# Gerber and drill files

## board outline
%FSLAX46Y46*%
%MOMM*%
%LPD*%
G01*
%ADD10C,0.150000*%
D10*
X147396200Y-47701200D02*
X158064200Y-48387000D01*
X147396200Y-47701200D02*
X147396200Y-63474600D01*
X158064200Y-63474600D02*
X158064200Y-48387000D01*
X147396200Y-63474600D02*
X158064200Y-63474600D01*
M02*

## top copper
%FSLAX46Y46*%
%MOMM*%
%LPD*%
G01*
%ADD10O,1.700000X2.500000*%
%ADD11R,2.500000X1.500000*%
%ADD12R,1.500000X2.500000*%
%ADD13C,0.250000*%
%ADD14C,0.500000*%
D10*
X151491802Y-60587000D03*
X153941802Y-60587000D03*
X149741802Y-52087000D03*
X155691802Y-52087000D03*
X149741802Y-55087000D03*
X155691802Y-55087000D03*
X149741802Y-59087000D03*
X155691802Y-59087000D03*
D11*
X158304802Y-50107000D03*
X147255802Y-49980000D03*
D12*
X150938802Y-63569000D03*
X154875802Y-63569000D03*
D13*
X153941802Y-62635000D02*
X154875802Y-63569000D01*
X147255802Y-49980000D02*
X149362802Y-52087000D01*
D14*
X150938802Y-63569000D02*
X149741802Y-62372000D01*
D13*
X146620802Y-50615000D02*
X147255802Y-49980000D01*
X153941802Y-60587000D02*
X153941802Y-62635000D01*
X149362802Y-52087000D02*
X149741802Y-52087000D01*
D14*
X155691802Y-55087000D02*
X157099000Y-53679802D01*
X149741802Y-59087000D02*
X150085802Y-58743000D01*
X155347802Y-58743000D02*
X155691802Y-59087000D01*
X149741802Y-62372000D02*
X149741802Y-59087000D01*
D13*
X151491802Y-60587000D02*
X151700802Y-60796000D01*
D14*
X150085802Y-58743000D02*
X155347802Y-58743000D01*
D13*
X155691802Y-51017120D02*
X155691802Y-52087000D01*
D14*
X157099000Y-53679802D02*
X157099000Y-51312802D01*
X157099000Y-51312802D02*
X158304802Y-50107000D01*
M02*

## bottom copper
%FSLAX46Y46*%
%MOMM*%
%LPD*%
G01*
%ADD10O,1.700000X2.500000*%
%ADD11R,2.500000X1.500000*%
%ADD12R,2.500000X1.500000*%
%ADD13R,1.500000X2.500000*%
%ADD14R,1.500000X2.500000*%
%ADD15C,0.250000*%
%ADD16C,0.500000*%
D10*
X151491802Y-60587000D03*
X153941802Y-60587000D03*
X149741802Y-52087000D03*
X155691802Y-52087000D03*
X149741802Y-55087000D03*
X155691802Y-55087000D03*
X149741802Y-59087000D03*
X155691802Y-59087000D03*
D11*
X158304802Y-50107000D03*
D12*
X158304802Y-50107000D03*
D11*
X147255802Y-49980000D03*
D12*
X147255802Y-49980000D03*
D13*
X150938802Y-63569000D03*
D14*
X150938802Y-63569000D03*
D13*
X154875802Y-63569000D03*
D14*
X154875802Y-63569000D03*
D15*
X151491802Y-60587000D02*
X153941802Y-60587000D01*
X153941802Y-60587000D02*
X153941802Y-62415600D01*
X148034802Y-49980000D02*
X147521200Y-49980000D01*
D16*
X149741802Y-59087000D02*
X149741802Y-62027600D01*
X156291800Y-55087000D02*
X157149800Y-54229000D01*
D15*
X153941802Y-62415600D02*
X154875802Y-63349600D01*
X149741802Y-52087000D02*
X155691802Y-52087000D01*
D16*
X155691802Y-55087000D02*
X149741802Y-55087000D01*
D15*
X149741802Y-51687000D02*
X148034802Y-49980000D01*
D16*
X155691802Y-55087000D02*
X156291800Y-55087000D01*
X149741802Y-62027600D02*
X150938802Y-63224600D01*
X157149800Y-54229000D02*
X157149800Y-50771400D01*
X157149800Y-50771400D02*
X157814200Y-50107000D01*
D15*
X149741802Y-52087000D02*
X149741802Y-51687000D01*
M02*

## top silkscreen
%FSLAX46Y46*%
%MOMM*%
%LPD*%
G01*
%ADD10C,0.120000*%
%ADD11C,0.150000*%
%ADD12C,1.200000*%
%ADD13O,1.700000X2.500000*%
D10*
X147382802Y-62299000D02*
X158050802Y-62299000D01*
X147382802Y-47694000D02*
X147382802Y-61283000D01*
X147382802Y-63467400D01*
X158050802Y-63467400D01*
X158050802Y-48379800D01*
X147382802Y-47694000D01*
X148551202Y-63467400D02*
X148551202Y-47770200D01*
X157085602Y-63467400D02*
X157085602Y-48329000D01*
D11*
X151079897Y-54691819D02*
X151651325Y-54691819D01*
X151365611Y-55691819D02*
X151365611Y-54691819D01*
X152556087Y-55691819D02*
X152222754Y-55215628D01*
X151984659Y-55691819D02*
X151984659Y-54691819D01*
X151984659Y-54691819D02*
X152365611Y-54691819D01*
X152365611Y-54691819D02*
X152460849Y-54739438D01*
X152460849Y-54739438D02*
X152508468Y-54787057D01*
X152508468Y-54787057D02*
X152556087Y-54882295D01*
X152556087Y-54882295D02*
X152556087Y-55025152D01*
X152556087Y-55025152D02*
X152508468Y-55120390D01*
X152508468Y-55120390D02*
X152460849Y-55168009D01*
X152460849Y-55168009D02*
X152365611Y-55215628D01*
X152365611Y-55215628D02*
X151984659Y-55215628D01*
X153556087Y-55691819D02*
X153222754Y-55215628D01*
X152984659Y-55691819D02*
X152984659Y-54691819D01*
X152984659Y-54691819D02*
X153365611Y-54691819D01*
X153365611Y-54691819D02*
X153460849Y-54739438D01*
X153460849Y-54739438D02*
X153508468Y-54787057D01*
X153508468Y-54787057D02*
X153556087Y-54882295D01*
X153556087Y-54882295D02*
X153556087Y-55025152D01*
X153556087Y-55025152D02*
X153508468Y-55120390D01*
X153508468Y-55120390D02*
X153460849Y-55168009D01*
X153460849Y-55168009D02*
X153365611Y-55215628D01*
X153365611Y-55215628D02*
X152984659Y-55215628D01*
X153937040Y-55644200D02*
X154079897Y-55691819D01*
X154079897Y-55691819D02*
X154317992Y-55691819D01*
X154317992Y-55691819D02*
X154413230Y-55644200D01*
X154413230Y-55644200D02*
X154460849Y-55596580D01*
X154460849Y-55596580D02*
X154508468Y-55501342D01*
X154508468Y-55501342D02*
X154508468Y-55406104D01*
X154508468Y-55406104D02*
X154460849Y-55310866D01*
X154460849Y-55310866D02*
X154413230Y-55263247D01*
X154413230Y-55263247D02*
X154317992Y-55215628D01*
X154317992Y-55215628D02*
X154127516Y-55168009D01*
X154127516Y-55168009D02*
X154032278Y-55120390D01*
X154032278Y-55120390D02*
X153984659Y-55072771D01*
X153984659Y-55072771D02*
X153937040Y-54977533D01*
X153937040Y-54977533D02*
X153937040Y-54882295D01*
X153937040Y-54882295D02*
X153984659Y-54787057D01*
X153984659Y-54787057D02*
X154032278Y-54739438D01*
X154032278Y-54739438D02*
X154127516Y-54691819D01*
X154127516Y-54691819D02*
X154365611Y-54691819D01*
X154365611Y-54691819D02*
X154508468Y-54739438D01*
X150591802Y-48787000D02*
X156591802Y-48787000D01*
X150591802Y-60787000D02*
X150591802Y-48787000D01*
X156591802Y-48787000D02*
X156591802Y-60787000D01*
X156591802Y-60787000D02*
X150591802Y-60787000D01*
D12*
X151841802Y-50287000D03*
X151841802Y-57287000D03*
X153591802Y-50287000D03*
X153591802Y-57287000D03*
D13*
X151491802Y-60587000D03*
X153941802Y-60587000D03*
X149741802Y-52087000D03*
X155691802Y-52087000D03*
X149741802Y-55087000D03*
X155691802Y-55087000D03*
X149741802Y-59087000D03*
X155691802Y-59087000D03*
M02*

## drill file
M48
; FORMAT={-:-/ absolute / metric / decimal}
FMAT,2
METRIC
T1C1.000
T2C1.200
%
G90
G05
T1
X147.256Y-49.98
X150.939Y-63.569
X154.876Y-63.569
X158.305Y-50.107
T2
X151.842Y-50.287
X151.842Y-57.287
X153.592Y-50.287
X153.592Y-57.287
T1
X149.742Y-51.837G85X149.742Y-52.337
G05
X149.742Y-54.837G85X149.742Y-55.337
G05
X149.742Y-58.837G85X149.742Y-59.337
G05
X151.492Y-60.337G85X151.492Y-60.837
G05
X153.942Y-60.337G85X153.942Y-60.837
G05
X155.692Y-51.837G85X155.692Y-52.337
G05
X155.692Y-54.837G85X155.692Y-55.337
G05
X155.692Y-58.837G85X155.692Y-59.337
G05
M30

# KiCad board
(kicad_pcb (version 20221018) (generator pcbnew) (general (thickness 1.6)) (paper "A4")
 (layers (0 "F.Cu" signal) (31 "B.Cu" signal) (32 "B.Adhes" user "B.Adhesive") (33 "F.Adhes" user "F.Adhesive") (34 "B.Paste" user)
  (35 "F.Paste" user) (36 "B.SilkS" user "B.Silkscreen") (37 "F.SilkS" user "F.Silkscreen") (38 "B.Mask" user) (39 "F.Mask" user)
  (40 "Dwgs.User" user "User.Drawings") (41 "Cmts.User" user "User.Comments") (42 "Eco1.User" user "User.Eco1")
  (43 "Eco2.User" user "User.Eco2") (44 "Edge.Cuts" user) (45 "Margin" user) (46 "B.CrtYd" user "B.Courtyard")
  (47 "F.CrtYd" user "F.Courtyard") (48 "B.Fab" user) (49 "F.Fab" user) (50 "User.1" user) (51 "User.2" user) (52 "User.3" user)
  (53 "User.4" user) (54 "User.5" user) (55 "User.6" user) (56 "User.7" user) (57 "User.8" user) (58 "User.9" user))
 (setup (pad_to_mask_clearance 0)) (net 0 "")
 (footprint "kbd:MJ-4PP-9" (layer "F.Cu") (at 153.591802 48.787)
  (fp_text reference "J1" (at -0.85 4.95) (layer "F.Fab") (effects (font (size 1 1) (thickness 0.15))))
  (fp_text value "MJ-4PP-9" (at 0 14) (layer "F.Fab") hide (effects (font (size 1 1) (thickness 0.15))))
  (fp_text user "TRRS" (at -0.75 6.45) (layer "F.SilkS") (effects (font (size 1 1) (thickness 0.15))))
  (fp_line (start -3 0) (end 3 0) (stroke (width 0.15) (type solid)) (layer "F.SilkS"))
  (fp_line (start -3 12) (end -3 0) (stroke (width 0.15) (type solid)) (layer "F.SilkS"))
  (fp_line (start 3 0) (end 3 12) (stroke (width 0.15) (type solid)) (layer "F.SilkS"))
  (fp_line (start 3 12) (end -3 12) (stroke (width 0.15) (type solid)) (layer "F.SilkS"))
  (pad "" np_thru_hole circle (at -1.75 1.5) (size 1.2 1.2) (drill 1.2) (layers "F&B.Cu" "*.Mask" "F.SilkS"))
  (pad "" np_thru_hole circle (at -1.75 8.5) (size 1.2 1.2) (drill 1.2) (layers "F&B.Cu" "*.Mask" "F.SilkS"))
  (pad "" np_thru_hole circle (at 0 1.5) (size 1.2 1.2) (drill 1.2) (layers "F&B.Cu" "*.Mask" "F.SilkS"))
  (pad "" np_thru_hole circle (at 0 8.5) (size 1.2 1.2) (drill 1.2) (layers "F&B.Cu" "*.Mask" "F.SilkS"))
  (pad "A" thru_hole oval (at -2.1 11.8) (size 1.7 2.5) (drill oval 1 1.5) (layers "*.Cu" "*.Mask" "F.SilkS") (clearance 0.15))
  (pad "A" thru_hole oval (at 0.35 11.8) (size 1.7 2.5) (drill oval 1 1.5) (layers "*.Cu" "*.Mask" "F.SilkS") (clearance 0.15))
  (pad "B" thru_hole oval (at -3.85 3.3) (size 1.7 2.5) (drill oval 1 1.5) (layers "*.Cu" "*.Mask" "F.SilkS"))
  (pad "B" thru_hole oval (at 2.1 3.3) (size 1.7 2.5) (drill oval 1 1.5) (layers "*.Cu" "*.Mask" "F.SilkS"))
  (pad "C" thru_hole oval (at -3.85 6.3) (size 1.7 2.5) (drill oval 1 1.5) (layers "*.Cu" "*.Mask" "F.SilkS"))
  (pad "C" thru_hole oval (at 2.1 6.3) (size 1.7 2.5) (drill oval 1 1.5) (layers "*.Cu" "*.Mask" "F.SilkS"))
  (pad "D" thru_hole oval (at -3.85 10.3) (size 1.7 2.5) (drill oval 1 1.5) (layers "*.Cu" "*.Mask" "F.SilkS") (clearance 0.15))
  (pad "D" thru_hole oval (at 2.1 10.3) (size 1.7 2.5) (drill oval 1 1.5) (layers "*.Cu" "*.Mask" "F.SilkS") (clearance 0.15)))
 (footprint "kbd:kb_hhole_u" (layer "F.Cu") (at 158.304802 50.107 -90)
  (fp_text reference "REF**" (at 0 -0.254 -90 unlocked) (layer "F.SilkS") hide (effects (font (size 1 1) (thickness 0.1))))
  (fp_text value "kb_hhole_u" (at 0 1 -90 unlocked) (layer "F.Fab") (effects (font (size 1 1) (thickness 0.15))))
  (pad "1" thru_hole rect (at 0 0 270) (size 1.5 2.5) (drill 1) (layers "*.Cu" "*.Adhes" "*.Mask"))
  (pad "1" smd rect (at 0 0 270) (size 1.5 2.5) (layers "*.Paste" "*.Mask" "B.Cu")))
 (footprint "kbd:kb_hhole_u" (layer "F.Cu") (at 147.255802 49.98 -90)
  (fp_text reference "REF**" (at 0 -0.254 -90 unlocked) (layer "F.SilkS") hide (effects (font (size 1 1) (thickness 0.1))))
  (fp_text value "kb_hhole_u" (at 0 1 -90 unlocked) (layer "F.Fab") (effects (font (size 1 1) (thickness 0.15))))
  (pad "1" thru_hole rect (at 0 0 270) (size 1.5 2.5) (drill 1) (layers "*.Cu" "*.Adhes" "*.Mask"))
  (pad "1" smd rect (at 0 0 270) (size 1.5 2.5) (layers "*.Paste" "*.Mask" "B.Cu")))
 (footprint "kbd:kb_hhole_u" (layer "F.Cu") (at 150.938802 63.569)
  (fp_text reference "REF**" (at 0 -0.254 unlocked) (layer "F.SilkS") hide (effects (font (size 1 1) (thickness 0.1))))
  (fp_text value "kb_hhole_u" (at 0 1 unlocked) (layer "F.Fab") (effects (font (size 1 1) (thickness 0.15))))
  (pad "1" thru_hole rect (at 0 0) (size 1.5 2.5) (drill 1) (layers "*.Cu" "*.Adhes" "*.Mask"))
  (pad "1" smd rect (at 0 0) (size 1.5 2.5) (layers "*.Paste" "*.Mask" "B.Cu")))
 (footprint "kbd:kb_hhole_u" (layer "F.Cu") (at 154.875802 63.569)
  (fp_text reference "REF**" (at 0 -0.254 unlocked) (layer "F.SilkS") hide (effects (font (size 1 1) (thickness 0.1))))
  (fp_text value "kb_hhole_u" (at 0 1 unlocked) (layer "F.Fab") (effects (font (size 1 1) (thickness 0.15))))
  (pad "1" thru_hole rect (at 0 0) (size 1.5 2.5) (drill 1) (layers "*.Cu" "*.Adhes" "*.Mask"))
  (pad "1" smd rect (at 0 0) (size 1.5 2.5) (layers "*.Paste" "*.Mask" "B.Cu")))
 (gr_line (start 147.382802 62.299) (end 158.050802 62.299) (stroke (width 0.12) (type default)) (layer "F.SilkS"))
 (gr_poly
  (pts (xy 147.382802 47.694) (xy 147.382802 61.283) (xy 147.382802 63.4674) (xy 158.050802 63.4674) (xy 158.050802 48.3798))
  (stroke (width 0.12) (type solid)) (fill none) (layer "F.SilkS"))
 (gr_line (start 148.551202 63.4674) (end 148.551202 47.7702) (stroke (width 0.12) (type default)) (layer "F.SilkS"))
 (gr_line (start 157.085602 63.4674) (end 157.085602 48.329) (stroke (width 0.12) (type default)) (layer "F.SilkS"))
 (gr_line (start 147.3962 47.7012) (end 158.0642 48.387) (stroke (width 0.15) (type default)) (layer "Edge.Cuts"))
 (gr_line (start 147.3962 47.7012) (end 147.3962 63.4746) (stroke (width 0.15) (type default)) (layer "Edge.Cuts"))
 (gr_line (start 158.0642 63.4746) (end 158.0642 48.387) (stroke (width 0.15) (type default)) (layer "Edge.Cuts"))
 (gr_line (start 147.3962 63.4746) (end 158.0642 63.4746) (stroke (width 0.15) (type default)) (layer "Edge.Cuts"))
 (segment (start 153.941802 62.635) (end 154.875802 63.569) (width 0.25) (layer "F.Cu") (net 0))
 (segment (start 147.255802 49.98) (end 149.362802 52.087) (width 0.25) (layer "F.Cu") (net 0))
 (segment (start 150.938802 63.569) (end 149.741802 62.372) (width 0.5) (layer "F.Cu") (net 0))
 (segment (start 146.620802 50.615) (end 147.255802 49.98) (width 0.25) (layer "F.Cu") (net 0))
 (segment (start 153.941802 60.587) (end 153.941802 62.635) (width 0.25) (layer "F.Cu") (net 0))
 (segment (start 149.362802 52.087) (end 149.741802 52.087) (width 0.25) (layer "F.Cu") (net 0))
 (segment (start 155.691802 55.087) (end 157.099 53.679802) (width 0.5) (layer "F.Cu") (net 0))
 (segment (start 149.741802 59.087) (end 150.085802 58.743) (width 0.5) (layer "F.Cu") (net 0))
 (segment (start 155.347802 58.743) (end 155.691802 59.087) (width 0.5) (layer "F.Cu") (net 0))
 (segment (start 149.741802 62.372) (end 149.741802 59.087) (width 0.5) (layer "F.Cu") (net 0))
 (segment (start 151.491802 60.587) (end 151.700802 60.796) (width 0.25) (layer "F.Cu") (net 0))
 (segment (start 150.085802 58.743) (end 155.347802 58.743) (width 0.5) (layer "F.Cu") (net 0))
 (segment (start 155.691802 51.01712) (end 155.691802 52.087) (width 0.25) (layer "F.Cu") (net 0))
 (segment (start 157.099 53.679802) (end 157.099 51.312802) (width 0.5) (layer "F.Cu") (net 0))
 (segment (start 157.099 51.312802) (end 158.304802 50.107) (width 0.5) (layer "F.Cu") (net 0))
 (segment (start 151.491802 60.587) (end 153.941802 60.587) (width 0.25) (layer "B.Cu") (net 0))
 (segment (start 153.941802 60.587) (end 153.941802 62.4156) (width 0.25) (layer "B.Cu") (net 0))
 (segment (start 148.034802 49.98) (end 147.5212 49.98) (width 0.25) (layer "B.Cu") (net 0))
 (segment (start 149.741802 59.087) (end 149.741802 62.0276) (width 0.5) (layer "B.Cu") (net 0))
 (segment (start 156.2918 55.087) (end 157.1498 54.229) (width 0.5) (layer "B.Cu") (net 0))
 (segment (start 153.941802 62.4156) (end 154.875802 63.3496) (width 0.25) (layer "B.Cu") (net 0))
 (segment (start 149.741802 52.087) (end 155.691802 52.087) (width 0.25) (layer "B.Cu") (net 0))
 (segment (start 155.691802 55.087) (end 149.741802 55.087) (width 0.5) (layer "B.Cu") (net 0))
 (segment (start 149.741802 51.687) (end 148.034802 49.98) (width 0.25) (layer "B.Cu") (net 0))
 (segment (start 155.691802 55.087) (end 156.2918 55.087) (width 0.5) (layer "B.Cu") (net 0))
 (segment (start 149.741802 62.0276) (end 150.938802 63.2246) (width 0.5) (layer "B.Cu") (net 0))
 (segment (start 157.1498 54.229) (end 157.1498 50.7714) (width 0.5) (layer "B.Cu") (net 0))
 (segment (start 157.1498 50.7714) (end 157.8142 50.107) (width 0.5) (layer "B.Cu") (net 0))
 (segment (start 149.741802 52.087) (end 149.741802 51.687) (width 0.25) (layer "B.Cu") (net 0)))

